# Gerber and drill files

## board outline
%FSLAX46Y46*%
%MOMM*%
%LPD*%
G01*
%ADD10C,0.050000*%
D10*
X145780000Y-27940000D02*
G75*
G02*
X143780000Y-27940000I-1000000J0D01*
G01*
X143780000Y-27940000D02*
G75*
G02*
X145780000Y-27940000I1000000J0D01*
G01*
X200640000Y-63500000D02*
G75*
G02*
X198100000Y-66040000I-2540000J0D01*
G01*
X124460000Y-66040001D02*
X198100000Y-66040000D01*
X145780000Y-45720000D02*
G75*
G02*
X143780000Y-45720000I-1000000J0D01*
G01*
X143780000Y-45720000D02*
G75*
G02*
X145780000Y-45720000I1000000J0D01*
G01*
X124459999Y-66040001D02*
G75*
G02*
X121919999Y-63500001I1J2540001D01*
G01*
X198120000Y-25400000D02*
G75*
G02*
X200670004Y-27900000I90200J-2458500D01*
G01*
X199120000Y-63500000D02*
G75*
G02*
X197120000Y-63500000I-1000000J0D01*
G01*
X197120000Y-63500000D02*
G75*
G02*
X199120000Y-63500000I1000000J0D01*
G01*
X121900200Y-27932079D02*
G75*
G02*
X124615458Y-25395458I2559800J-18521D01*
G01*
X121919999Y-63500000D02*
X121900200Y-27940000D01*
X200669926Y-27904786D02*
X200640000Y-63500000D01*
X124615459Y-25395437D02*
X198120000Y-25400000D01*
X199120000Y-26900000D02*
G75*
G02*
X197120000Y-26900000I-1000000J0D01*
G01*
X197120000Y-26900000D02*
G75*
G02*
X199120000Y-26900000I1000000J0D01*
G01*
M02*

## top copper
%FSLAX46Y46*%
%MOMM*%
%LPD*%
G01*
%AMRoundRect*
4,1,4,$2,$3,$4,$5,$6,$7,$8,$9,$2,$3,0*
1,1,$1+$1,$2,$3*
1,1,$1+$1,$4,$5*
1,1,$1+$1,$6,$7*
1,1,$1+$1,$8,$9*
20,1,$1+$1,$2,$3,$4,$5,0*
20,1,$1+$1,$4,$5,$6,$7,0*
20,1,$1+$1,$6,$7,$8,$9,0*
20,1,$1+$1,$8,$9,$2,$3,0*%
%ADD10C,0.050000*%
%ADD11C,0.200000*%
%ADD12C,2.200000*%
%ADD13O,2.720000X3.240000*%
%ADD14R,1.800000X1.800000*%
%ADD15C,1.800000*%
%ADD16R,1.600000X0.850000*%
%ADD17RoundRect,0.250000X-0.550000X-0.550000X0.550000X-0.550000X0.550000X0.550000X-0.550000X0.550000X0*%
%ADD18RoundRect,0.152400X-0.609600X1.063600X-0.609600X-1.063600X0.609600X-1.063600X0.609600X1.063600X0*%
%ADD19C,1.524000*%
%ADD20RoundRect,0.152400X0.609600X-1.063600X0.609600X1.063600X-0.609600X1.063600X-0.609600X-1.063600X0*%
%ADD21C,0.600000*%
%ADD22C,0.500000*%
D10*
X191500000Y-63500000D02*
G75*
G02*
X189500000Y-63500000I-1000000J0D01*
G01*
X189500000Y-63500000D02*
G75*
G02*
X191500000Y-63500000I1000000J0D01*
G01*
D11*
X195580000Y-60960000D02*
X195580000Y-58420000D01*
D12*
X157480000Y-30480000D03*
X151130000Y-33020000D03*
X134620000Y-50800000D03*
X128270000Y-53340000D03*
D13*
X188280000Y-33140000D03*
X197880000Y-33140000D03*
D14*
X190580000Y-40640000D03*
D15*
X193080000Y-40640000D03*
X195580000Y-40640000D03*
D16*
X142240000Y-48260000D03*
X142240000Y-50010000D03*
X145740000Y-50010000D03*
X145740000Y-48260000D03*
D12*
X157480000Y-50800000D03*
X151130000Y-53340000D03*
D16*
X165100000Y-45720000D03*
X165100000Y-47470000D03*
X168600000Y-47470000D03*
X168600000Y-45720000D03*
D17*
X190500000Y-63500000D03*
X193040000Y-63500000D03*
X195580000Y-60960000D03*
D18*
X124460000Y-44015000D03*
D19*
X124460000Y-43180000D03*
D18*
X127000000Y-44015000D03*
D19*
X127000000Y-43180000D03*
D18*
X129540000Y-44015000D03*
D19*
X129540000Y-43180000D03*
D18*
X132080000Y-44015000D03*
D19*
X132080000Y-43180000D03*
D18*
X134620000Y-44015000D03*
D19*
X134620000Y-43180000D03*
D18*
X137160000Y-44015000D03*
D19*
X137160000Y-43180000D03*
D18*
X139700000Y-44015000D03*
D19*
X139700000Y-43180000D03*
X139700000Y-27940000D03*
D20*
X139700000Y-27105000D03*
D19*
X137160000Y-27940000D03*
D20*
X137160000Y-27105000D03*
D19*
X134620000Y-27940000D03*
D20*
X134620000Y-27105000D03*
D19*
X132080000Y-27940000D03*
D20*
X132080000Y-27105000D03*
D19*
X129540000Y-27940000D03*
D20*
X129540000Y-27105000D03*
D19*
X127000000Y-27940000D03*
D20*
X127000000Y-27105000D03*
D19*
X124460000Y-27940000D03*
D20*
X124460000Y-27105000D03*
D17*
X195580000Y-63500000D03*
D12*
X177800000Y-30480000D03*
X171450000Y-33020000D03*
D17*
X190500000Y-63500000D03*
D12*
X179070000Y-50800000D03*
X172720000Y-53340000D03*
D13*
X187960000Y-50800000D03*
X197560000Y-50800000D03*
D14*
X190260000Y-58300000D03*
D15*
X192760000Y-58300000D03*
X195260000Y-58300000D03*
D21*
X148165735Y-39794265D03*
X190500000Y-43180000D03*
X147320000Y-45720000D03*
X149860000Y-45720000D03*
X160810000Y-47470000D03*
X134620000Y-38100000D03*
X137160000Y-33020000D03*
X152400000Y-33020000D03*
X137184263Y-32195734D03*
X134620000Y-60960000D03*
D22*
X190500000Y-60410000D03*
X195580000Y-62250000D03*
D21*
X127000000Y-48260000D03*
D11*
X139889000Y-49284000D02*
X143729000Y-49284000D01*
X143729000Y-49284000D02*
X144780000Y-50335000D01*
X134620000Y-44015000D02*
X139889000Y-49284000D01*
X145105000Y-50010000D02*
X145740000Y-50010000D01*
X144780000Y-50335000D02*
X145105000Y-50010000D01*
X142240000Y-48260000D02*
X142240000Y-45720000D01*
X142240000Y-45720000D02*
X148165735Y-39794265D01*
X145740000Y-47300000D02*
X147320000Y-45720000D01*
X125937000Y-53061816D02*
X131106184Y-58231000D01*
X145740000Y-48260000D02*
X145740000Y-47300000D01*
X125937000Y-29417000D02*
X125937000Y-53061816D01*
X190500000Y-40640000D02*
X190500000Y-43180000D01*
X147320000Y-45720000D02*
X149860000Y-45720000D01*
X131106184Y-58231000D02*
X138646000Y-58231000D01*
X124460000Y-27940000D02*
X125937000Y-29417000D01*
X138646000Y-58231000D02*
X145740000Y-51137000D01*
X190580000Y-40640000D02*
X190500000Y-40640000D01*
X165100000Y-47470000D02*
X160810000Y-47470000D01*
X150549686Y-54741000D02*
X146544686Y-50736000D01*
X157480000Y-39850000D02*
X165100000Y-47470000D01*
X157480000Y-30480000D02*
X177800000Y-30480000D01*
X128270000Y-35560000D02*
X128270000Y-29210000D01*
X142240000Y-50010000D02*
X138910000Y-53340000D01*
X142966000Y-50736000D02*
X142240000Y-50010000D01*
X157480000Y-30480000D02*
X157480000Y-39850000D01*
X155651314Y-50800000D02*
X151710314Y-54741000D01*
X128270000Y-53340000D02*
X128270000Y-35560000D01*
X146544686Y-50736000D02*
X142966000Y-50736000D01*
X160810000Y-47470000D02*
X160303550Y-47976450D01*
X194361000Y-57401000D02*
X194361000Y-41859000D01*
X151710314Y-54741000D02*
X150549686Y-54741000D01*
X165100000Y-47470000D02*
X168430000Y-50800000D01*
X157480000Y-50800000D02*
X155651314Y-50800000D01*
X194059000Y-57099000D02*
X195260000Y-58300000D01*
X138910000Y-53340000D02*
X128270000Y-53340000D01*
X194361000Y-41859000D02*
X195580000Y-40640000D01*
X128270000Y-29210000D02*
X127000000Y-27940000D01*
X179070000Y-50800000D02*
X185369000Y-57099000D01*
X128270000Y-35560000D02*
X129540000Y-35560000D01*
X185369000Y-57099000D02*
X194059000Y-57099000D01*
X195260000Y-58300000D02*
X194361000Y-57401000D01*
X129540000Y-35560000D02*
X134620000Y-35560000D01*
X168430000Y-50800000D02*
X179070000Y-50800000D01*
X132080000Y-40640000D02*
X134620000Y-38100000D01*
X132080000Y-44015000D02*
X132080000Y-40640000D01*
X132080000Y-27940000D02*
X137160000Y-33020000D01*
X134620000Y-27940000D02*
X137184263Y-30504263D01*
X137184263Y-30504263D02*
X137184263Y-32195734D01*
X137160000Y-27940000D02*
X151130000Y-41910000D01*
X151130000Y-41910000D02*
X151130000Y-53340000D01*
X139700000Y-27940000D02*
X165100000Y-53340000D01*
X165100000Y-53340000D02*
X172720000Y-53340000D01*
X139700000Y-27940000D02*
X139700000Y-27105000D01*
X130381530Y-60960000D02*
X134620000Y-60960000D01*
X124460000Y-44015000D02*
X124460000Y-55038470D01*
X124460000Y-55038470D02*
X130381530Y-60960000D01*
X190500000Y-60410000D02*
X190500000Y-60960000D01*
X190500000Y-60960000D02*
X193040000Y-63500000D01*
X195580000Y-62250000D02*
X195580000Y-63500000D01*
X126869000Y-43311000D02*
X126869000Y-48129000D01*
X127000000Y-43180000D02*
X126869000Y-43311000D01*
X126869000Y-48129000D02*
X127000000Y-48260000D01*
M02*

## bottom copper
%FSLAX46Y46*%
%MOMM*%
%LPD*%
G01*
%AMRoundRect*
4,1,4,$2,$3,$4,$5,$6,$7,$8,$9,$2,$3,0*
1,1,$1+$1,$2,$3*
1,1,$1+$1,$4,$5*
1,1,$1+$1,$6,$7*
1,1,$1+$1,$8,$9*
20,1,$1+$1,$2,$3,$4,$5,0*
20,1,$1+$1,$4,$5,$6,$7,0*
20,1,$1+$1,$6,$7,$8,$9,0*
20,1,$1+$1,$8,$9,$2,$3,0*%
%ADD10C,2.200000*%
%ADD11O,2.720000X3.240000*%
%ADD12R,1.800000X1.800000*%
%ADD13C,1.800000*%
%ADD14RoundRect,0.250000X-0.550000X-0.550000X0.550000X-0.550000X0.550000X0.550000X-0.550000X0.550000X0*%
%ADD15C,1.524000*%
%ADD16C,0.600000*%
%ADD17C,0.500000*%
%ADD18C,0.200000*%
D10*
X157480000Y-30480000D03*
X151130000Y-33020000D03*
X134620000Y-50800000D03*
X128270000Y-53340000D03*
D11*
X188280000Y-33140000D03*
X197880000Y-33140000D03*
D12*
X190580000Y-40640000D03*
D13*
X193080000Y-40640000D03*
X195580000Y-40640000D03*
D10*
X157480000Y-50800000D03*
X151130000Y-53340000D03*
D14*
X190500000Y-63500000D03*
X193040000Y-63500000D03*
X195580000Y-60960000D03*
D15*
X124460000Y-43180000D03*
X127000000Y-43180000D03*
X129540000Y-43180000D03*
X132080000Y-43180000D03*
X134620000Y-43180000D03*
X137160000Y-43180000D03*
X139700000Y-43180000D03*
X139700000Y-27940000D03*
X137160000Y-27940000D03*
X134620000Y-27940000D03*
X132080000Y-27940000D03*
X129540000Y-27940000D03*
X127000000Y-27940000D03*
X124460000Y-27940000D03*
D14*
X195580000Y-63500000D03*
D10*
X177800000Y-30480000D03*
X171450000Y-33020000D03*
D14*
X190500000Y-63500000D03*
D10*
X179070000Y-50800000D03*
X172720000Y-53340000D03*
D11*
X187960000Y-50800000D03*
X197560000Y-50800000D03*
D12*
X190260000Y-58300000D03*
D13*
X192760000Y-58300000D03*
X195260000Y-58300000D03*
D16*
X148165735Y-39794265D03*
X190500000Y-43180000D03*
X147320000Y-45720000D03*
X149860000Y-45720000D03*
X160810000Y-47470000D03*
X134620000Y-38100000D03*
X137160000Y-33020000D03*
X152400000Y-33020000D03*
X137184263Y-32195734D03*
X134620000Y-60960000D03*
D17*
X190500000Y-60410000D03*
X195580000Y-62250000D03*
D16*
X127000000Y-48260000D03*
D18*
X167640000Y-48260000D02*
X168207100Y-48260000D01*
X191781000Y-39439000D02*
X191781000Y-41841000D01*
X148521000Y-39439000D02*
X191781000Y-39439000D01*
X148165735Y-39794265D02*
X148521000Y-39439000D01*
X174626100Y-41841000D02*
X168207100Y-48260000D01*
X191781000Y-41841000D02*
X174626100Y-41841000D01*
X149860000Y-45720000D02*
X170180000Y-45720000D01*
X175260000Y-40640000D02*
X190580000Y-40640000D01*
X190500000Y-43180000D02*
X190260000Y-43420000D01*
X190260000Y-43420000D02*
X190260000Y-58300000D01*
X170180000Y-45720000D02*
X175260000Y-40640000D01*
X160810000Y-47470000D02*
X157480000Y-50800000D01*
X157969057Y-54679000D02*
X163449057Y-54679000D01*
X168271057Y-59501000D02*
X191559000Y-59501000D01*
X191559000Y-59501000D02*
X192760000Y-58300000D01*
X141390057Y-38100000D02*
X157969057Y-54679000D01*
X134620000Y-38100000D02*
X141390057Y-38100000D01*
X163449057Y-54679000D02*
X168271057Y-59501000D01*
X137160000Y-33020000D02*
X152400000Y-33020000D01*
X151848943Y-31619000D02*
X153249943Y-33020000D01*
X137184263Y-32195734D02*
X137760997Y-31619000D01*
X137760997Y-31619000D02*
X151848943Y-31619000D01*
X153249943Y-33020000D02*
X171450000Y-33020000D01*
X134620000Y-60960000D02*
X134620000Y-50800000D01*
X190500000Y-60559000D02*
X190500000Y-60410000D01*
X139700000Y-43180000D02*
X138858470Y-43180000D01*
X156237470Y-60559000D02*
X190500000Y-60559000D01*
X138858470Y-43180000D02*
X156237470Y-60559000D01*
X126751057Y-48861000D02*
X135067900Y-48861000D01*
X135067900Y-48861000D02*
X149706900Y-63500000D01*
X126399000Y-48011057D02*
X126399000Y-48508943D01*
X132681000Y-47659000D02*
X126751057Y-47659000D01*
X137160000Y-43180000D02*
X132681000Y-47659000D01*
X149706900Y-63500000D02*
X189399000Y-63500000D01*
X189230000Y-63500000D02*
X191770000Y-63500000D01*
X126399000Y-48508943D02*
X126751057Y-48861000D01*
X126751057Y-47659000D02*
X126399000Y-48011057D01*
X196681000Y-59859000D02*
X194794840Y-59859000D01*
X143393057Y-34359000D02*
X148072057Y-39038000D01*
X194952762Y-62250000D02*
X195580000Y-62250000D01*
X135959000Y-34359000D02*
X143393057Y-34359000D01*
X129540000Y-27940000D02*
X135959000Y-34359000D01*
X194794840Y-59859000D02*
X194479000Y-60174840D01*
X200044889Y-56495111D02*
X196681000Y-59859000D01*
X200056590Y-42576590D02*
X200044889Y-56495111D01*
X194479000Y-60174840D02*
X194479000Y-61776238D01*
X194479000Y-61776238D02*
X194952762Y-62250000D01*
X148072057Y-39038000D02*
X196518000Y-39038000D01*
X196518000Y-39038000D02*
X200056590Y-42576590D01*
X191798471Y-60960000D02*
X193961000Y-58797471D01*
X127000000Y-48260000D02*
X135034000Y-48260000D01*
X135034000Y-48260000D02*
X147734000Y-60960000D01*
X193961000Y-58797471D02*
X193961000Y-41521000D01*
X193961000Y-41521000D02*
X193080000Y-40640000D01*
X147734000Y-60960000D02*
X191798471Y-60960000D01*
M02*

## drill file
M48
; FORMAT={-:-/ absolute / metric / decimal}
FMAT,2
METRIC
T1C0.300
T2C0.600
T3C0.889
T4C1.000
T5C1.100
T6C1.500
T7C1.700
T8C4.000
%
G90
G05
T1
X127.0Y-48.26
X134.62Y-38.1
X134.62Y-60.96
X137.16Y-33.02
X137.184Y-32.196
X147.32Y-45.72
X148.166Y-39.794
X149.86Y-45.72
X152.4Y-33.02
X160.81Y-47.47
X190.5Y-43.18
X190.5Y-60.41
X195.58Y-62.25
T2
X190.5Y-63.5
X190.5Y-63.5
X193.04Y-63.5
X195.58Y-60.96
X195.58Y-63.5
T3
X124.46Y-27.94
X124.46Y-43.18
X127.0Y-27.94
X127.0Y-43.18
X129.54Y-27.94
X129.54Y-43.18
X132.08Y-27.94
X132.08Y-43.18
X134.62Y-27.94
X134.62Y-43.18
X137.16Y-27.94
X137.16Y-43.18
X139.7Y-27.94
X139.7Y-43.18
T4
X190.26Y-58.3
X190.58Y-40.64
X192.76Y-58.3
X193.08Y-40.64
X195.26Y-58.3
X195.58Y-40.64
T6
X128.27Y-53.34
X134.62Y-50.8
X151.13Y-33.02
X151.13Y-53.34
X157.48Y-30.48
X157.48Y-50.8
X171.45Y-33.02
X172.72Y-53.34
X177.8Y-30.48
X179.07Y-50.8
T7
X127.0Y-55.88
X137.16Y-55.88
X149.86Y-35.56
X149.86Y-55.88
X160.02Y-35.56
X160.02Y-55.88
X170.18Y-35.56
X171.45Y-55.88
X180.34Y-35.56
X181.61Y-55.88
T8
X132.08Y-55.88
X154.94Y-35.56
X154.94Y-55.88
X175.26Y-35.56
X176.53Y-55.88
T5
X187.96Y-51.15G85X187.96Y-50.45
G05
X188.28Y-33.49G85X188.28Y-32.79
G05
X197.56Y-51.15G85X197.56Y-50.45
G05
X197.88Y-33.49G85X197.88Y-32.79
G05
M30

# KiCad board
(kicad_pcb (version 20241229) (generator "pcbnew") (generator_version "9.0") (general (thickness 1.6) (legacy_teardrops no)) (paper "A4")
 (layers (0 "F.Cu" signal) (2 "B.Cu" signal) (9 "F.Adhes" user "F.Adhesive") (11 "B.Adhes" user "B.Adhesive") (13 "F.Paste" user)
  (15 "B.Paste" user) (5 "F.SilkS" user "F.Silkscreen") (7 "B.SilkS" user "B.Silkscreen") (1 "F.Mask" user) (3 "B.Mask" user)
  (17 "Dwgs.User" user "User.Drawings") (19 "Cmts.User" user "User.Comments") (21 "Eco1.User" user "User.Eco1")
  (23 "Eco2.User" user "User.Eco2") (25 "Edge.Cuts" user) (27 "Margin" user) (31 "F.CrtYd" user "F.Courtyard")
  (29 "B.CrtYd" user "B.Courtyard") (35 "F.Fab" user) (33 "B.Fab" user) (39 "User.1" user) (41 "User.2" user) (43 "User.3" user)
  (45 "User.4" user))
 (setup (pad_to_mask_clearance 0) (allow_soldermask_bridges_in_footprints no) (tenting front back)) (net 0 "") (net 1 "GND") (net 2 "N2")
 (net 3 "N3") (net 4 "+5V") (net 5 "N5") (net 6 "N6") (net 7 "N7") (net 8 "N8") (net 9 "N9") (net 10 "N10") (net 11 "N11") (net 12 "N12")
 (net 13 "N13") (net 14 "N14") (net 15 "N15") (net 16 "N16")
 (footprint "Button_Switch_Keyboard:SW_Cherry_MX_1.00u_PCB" (layer "F.Cu") (at 157.48 30.48)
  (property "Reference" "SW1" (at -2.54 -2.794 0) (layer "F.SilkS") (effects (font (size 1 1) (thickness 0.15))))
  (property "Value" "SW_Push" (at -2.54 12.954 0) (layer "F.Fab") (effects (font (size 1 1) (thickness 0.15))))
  (pad "" np_thru_hole circle (at -7.62 5.08) (size 1.7 1.7) (drill 1.7) (layers "*.Cu" "*.Mask"))
  (pad "" np_thru_hole circle (at -2.54 5.08) (size 4 4) (drill 4) (layers "*.Cu" "*.Mask"))
  (pad "" np_thru_hole circle (at 2.54 5.08) (size 1.7 1.7) (drill 1.7) (layers "*.Cu" "*.Mask"))
  (pad "1" thru_hole circle (at 0 0) (size 2.2 2.2) (drill 1.5) (layers "*.Cu" "*.Mask") (remove_unused_layers no) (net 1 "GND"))
  (pad "2" thru_hole circle (at -6.35 2.54) (size 2.2 2.2) (drill 1.5) (layers "*.Cu" "*.Mask") (remove_unused_layers no) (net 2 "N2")))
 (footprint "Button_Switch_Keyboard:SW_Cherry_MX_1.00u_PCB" (layer "F.Cu") (at 134.62 50.8)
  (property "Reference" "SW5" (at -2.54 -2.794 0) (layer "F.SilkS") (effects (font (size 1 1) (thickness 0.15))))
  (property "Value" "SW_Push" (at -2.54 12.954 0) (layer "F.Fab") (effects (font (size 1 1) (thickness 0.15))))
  (pad "" np_thru_hole circle (at -7.62 5.08) (size 1.7 1.7) (drill 1.7) (layers "*.Cu" "*.Mask"))
  (pad "" np_thru_hole circle (at -2.54 5.08) (size 4 4) (drill 4) (layers "*.Cu" "*.Mask"))
  (pad "" np_thru_hole circle (at 2.54 5.08) (size 1.7 1.7) (drill 1.7) (layers "*.Cu" "*.Mask"))
  (pad "1" thru_hole circle (at 0 0) (size 2.2 2.2) (drill 1.5) (layers "*.Cu" "*.Mask") (remove_unused_layers no) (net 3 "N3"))
  (pad "2" thru_hole circle (at -6.35 2.54) (size 2.2 2.2) (drill 1.5) (layers "*.Cu" "*.Mask") (remove_unused_layers no) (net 1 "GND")))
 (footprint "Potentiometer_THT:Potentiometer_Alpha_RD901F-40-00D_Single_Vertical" (layer "F.Cu") (at 190.58 40.64 90)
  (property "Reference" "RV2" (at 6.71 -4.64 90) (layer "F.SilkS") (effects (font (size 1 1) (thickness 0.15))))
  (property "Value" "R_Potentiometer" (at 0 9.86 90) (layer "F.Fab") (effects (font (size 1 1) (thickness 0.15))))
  (pad "" thru_hole oval (at 7.5 -2.3 180) (size 2.72 3.24) (drill oval 1.1 1.8) (layers "*.Cu" "*.Mask") (remove_unused_layers no))
  (pad "" thru_hole oval (at 7.5 7.3 180) (size 2.72 3.24) (drill oval 1.1 1.8) (layers "*.Cu" "*.Mask") (remove_unused_layers no))
  (pad "1" thru_hole rect (at 0 0 180) (size 1.8 1.8) (drill 1) (layers "*.Cu" "*.Mask") (remove_unused_layers no) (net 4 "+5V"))
  (pad "2" thru_hole circle (at 0 2.5 180) (size 1.8 1.8) (drill 1) (layers "*.Cu" "*.Mask") (remove_unused_layers no) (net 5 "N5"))
  (pad "3" thru_hole circle (at 0 5 180) (size 1.8 1.8) (drill 1) (layers "*.Cu" "*.Mask") (remove_unused_layers no) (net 1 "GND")))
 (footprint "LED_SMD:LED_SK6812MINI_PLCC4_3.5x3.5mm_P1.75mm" (layer "F.Cu") (at 143.99 49.135)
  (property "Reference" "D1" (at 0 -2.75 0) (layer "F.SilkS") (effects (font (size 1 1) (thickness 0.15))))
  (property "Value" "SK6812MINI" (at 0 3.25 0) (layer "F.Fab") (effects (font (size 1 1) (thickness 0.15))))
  (pad "1" smd rect (at -1.75 -0.875) (size 1.6 0.85) (layers "F.Cu" "F.Mask" "F.Paste") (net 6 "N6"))
  (pad "2" smd rect (at -1.75 0.875) (size 1.6 0.85) (layers "F.Cu" "F.Mask" "F.Paste") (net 1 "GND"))
  (pad "3" smd rect (at 1.75 0.875) (size 1.6 0.85) (layers "F.Cu" "F.Mask" "F.Paste") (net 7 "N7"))
  (pad "4" smd rect (at 1.75 -0.875) (size 1.6 0.85) (layers "F.Cu" "F.Mask" "F.Paste") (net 4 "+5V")))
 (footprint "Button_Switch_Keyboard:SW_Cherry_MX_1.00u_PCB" (layer "F.Cu") (at 157.48 50.8)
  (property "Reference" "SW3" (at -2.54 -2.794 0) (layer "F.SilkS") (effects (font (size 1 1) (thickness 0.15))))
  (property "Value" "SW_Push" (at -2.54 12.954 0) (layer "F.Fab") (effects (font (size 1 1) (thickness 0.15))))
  (pad "" np_thru_hole circle (at -7.62 5.08) (size 1.7 1.7) (drill 1.7) (layers "*.Cu" "*.Mask"))
  (pad "" np_thru_hole circle (at -2.54 5.08) (size 4 4) (drill 4) (layers "*.Cu" "*.Mask"))
  (pad "" np_thru_hole circle (at 2.54 5.08) (size 1.7 1.7) (drill 1.7) (layers "*.Cu" "*.Mask"))
  (pad "1" thru_hole circle (at 0 0) (size 2.2 2.2) (drill 1.5) (layers "*.Cu" "*.Mask") (remove_unused_layers no) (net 1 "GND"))
  (pad "2" thru_hole circle (at -6.35 2.54) (size 2.2 2.2) (drill 1.5) (layers "*.Cu" "*.Mask") (remove_unused_layers no) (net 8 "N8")))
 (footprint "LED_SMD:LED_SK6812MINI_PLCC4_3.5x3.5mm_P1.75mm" (layer "F.Cu") (at 166.85 46.595)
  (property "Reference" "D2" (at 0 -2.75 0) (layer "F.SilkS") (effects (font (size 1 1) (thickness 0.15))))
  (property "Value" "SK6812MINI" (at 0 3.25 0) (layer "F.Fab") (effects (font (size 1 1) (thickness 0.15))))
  (pad "1" smd rect (at -1.75 -0.875) (size 1.6 0.85) (layers "F.Cu" "F.Mask" "F.Paste") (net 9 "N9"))
  (pad "2" smd rect (at -1.75 0.875) (size 1.6 0.85) (layers "F.Cu" "F.Mask" "F.Paste") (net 1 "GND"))
  (pad "3" smd rect (at 1.75 0.875) (size 1.6 0.85) (layers "F.Cu" "F.Mask" "F.Paste") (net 6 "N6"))
  (pad "4" smd rect (at 1.75 -0.875) (size 1.6 0.85) (layers "F.Cu" "F.Mask" "F.Paste") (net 4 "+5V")))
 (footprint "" (layer "F.Cu") (at 190.5 63.5)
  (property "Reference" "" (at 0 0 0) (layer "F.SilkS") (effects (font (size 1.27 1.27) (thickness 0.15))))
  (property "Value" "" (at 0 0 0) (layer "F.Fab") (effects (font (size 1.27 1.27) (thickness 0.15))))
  (pad "1" thru_hole roundrect (at 0 0) (size 1.6 1.6) (drill 0.6) (layers "*.Cu" "*.Mask") (remove_unused_layers no)
   (roundrect_rratio 0.15625)))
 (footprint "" (layer "F.Cu") (at 193.04 63.5)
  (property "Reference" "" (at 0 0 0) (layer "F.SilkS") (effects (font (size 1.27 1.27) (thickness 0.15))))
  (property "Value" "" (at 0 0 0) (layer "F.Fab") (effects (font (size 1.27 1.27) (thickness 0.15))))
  (pad "1" thru_hole roundrect (at 0 0) (size 1.6 1.6) (drill 0.6) (layers "*.Cu" "*.Mask") (remove_unused_layers no)
   (roundrect_rratio 0.15625)))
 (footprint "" (layer "F.Cu") (at 195.58 60.96)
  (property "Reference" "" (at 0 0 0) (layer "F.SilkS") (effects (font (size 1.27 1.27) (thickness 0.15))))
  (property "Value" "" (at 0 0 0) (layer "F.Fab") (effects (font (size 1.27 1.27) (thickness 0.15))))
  (pad "1" thru_hole roundrect (at 0 0) (size 1.6 1.6) (drill 0.6) (layers "*.Cu" "*.Mask") (remove_unused_layers no)
   (roundrect_rratio 0.15625)))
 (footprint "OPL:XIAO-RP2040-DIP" (layer "F.Cu") (at 132.08 35.56 90)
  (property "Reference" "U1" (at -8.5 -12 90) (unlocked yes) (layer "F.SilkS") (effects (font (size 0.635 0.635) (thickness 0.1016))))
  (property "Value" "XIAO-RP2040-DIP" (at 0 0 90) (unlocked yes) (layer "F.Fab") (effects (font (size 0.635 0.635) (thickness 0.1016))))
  (pad "1" smd roundrect (at -8.455 -7.62 270) (size 2.432 1.524) (layers "F.Cu" "F.Mask") (roundrect_rratio 0.1) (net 3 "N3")
   (thermal_bridge_angle 45))
  (pad "1" thru_hole circle (at -7.62 -7.62 270) (size 1.524 1.524) (drill 0.889) (layers "*.Cu" "*.Mask") (remove_unused_layers no)
   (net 3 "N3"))
  (pad "2" smd roundrect (at -8.455 -5.08 270) (size 2.432 1.524) (layers "F.Cu" "F.Mask") (roundrect_rratio 0.1) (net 5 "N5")
   (thermal_bridge_angle 45))
  (pad "2" thru_hole circle (at -7.62 -5.08 270) (size 1.524 1.524) (drill 0.889) (layers "*.Cu" "*.Mask") (remove_unused_layers no)
   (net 5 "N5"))
  (pad "3" smd roundrect (at -8.455 -2.54 270) (size 2.432 1.524) (layers "F.Cu" "F.Mask") (roundrect_rratio 0.1) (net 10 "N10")
   (thermal_bridge_angle 45))
  (pad "3" thru_hole circle (at -7.62 -2.54 270) (size 1.524 1.524) (drill 0.889) (layers "*.Cu" "*.Mask") (remove_unused_layers no)
   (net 10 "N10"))
  (pad "4" smd roundrect (at -8.455 0 270) (size 2.432 1.524) (layers "F.Cu" "F.Mask") (roundrect_rratio 0.1) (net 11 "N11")
   (thermal_bridge_angle 45))
  (pad "4" thru_hole circle (at -7.62 0 270) (size 1.524 1.524) (drill 0.889) (layers "*.Cu" "*.Mask") (remove_unused_layers no)
   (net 11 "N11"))
  (pad "5" smd roundrect (at -8.455 2.54 270) (size 2.432 1.524) (layers "F.Cu" "F.Mask") (roundrect_rratio 0.1) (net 7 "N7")
   (thermal_bridge_angle 45))
  (pad "5" thru_hole circle (at -7.62 2.54 270) (size 1.524 1.524) (drill 0.889) (layers "*.Cu" "*.Mask") (remove_unused_layers no)
   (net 7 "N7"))
  (pad "6" smd roundrect (at -8.455 5.08 270) (size 2.432 1.524) (layers "F.Cu" "F.Mask") (roundrect_rratio 0.1) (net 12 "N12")
   (thermal_bridge_angle 45))
  (pad "6" thru_hole circle (at -7.62 5.08 270) (size 1.524 1.524) (drill 0.889) (layers "*.Cu" "*.Mask") (remove_unused_layers no)
   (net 12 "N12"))
  (pad "7" smd roundrect (at -8.455 7.62 270) (size 2.432 1.524) (layers "F.Cu" "F.Mask") (roundrect_rratio 0.1) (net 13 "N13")
   (thermal_bridge_angle 45))
  (pad "7" thru_hole circle (at -7.62 7.62 270) (size 1.524 1.524) (drill 0.889) (layers "*.Cu" "*.Mask") (remove_unused_layers no)
   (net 13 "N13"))
  (pad "8" thru_hole circle (at 7.62 7.62 90) (size 1.524 1.524) (drill 0.889) (layers "*.Cu" "*.Mask") (remove_unused_layers no)
   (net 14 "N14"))
  (pad "8" smd roundrect (at 8.455 7.62 90) (size 2.432 1.524) (layers "F.Cu" "F.Mask") (roundrect_rratio 0.1) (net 14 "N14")
   (thermal_bridge_angle 45))
  (pad "9" thru_hole circle (at 7.62 5.08 90) (size 1.524 1.524) (drill 0.889) (layers "*.Cu" "*.Mask") (remove_unused_layers no)
   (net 8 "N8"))
  (pad "9" smd roundrect (at 8.455 5.08 90) (size 2.432 1.524) (layers "F.Cu" "F.Mask") (roundrect_rratio 0.1) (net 8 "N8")
   (thermal_bridge_angle 45))
  (pad "10" thru_hole circle (at 7.62 2.54 90) (size 1.524 1.524) (drill 0.889) (layers "*.Cu" "*.Mask") (remove_unused_layers no)
   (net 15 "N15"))
  (pad "10" smd roundrect (at 8.455 2.54 90) (size 2.432 1.524) (layers "F.Cu" "F.Mask") (roundrect_rratio 0.1) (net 15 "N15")
   (thermal_bridge_angle 45))
  (pad "11" thru_hole circle (at 7.62 0 90) (size 1.524 1.524) (drill 0.889) (layers "*.Cu" "*.Mask") (remove_unused_layers no) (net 2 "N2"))
  (pad "11" smd roundrect (at 8.455 0 90) (size 2.432 1.524) (layers "F.Cu" "F.Mask") (roundrect_rratio 0.1) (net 2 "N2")
   (thermal_bridge_angle 45))
  (pad "12" thru_hole circle (at 7.62 -2.54 90) (size 1.524 1.524) (drill 0.889) (layers "*.Cu" "*.Mask") (remove_unused_layers no)
   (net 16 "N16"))
  (pad "12" smd roundrect (at 8.455 -2.54 90) (size 2.432 1.524) (layers "F.Cu" "F.Mask") (roundrect_rratio 0.1) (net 16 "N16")
   (thermal_bridge_angle 45))
  (pad "13" thru_hole circle (at 7.62 -5.08 90) (size 1.524 1.524) (drill 0.889) (layers "*.Cu" "*.Mask") (remove_unused_layers no)
   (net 1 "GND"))
  (pad "13" smd roundrect (at 8.455 -5.08 90) (size 2.432 1.524) (layers "F.Cu" "F.Mask") (roundrect_rratio 0.1) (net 1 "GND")
   (thermal_bridge_angle 45))
  (pad "14" thru_hole circle (at 7.62 -7.62 90) (size 1.524 1.524) (drill 0.889) (layers "*.Cu" "*.Mask") (remove_unused_layers no)
   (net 4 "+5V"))
  (pad "14" smd roundrect (at 8.455 -7.62 90) (size 2.432 1.524) (layers "F.Cu" "F.Mask") (roundrect_rratio 0.1) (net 4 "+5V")
   (thermal_bridge_angle 45)))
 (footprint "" (layer "F.Cu") (at 195.58 63.5)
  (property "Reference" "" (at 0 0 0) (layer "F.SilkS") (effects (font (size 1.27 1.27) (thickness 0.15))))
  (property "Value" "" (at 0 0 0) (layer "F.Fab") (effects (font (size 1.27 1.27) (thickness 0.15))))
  (pad "1" thru_hole roundrect (at 0 0) (size 1.6 1.6) (drill 0.6) (layers "*.Cu" "*.Mask") (remove_unused_layers no)
   (roundrect_rratio 0.15625)))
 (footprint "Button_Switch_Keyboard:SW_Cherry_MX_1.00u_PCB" (layer "F.Cu") (at 177.8 30.48)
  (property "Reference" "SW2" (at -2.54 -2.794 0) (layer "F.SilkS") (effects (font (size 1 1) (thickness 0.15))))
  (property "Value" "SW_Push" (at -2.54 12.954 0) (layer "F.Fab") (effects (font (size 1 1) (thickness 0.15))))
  (pad "" np_thru_hole circle (at -7.62 5.08) (size 1.7 1.7) (drill 1.7) (layers "*.Cu" "*.Mask"))
  (pad "" np_thru_hole circle (at -2.54 5.08) (size 4 4) (drill 4) (layers "*.Cu" "*.Mask"))
  (pad "" np_thru_hole circle (at 2.54 5.08) (size 1.7 1.7) (drill 1.7) (layers "*.Cu" "*.Mask"))
  (pad "1" thru_hole circle (at 0 0) (size 2.2 2.2) (drill 1.5) (layers "*.Cu" "*.Mask") (remove_unused_layers no) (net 1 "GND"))
  (pad "2" thru_hole circle (at -6.35 2.54) (size 2.2 2.2) (drill 1.5) (layers "*.Cu" "*.Mask") (remove_unused_layers no) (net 15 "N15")))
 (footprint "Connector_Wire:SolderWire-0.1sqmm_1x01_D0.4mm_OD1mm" (layer "F.Cu") (at 190.5 63.5)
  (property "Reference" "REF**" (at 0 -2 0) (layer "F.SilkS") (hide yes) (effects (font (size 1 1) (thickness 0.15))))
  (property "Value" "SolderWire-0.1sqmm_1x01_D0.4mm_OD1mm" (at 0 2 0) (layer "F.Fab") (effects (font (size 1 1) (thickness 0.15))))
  (pad "1" thru_hole roundrect (at 0 0) (size 1.6 1.6) (drill 0.6) (layers "*.Cu" "*.Mask") (remove_unused_layers no)
   (roundrect_rratio 0.15625)))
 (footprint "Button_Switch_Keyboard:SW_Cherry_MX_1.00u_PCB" (layer "F.Cu") (at 179.07 50.8)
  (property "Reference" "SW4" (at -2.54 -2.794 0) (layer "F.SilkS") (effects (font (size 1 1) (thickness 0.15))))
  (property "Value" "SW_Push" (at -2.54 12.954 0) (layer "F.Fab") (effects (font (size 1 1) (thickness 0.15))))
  (pad "" np_thru_hole circle (at -7.62 5.08) (size 1.7 1.7) (drill 1.7) (layers "*.Cu" "*.Mask"))
  (pad "" np_thru_hole circle (at -2.54 5.08) (size 4 4) (drill 4) (layers "*.Cu" "*.Mask"))
  (pad "" np_thru_hole circle (at 2.54 5.08) (size 1.7 1.7) (drill 1.7) (layers "*.Cu" "*.Mask"))
  (pad "1" thru_hole circle (at 0 0) (size 2.2 2.2) (drill 1.5) (layers "*.Cu" "*.Mask") (remove_unused_layers no) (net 1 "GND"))
  (pad "2" thru_hole circle (at -6.35 2.54) (size 2.2 2.2) (drill 1.5) (layers "*.Cu" "*.Mask") (remove_unused_layers no) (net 14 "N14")))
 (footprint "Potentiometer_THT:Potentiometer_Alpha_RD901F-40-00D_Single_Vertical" (layer "F.Cu") (at 190.26 58.3 90)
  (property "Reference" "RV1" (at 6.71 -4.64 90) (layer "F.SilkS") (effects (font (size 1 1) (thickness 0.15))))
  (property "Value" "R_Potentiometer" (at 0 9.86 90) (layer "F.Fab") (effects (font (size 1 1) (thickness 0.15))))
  (pad "" thru_hole oval (at 7.5 -2.3 180) (size 2.72 3.24) (drill oval 1.1 1.8) (layers "*.Cu" "*.Mask") (remove_unused_layers no))
  (pad "" thru_hole oval (at 7.5 7.3 180) (size 2.72 3.24) (drill oval 1.1 1.8) (layers "*.Cu" "*.Mask") (remove_unused_layers no))
  (pad "1" thru_hole rect (at 0 0 180) (size 1.8 1.8) (drill 1) (layers "*.Cu" "*.Mask") (remove_unused_layers no) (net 4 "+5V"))
  (pad "2" thru_hole circle (at 0 2.5 180) (size 1.8 1.8) (drill 1) (layers "*.Cu" "*.Mask") (remove_unused_layers no) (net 11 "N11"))
  (pad "3" thru_hole circle (at 0 5 180) (size 1.8 1.8) (drill 1) (layers "*.Cu" "*.Mask") (remove_unused_layers no) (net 1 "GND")))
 (gr_circle (center 190.5 63.5) (end 191.5 63.5) (stroke (width 0.05) (type solid)) (fill no) (layer "F.Cu") (net 12))
 (gr_line (start 195.58 60.96) (end 195.58 58.42) (stroke (width 0.2) (type default)) (layer "F.Cu") (net 1))
 (gr_circle (center 144.78 27.94) (end 145.78 27.94) (stroke (width 0.05) (type solid)) (fill no) (layer "Edge.Cuts"))
 (gr_arc (start 200.64 63.5) (mid 199.896051 65.296051) (end 198.1 66.04) (stroke (width 0.05) (type solid)) (layer "Edge.Cuts"))
 (gr_line (start 124.46 66.040001) (end 198.1 66.04) (stroke (width 0.05) (type default)) (layer "Edge.Cuts"))
 (gr_circle (center 144.78 45.72) (end 145.78 45.72) (stroke (width 0.05) (type solid)) (fill no) (layer "Edge.Cuts"))
 (gr_arc (start 124.459999 66.040001) (mid 122.663948 65.296052) (end 121.919999 63.500001) (stroke (width 0.05) (type solid))
  (layer "Edge.Cuts"))
 (gr_arc (start 198.12 25.4) (mid 199.920193 26.089807) (end 200.67 27.9) (stroke (width 0.05) (type solid)) (layer "Edge.Cuts"))
 (gr_circle (center 198.12 63.5) (end 199.12 63.5) (stroke (width 0.05) (type solid)) (fill no) (layer "Edge.Cuts"))
 (gr_arc (start 121.9002 27.932079) (mid 122.712473 26.08) (end 124.615459 25.395437) (stroke (width 0.05) (type solid)) (layer "Edge.Cuts"))
 (gr_line (start 121.919999 63.5) (end 121.9002 27.94) (stroke (width 0.05) (type default)) (layer "Edge.Cuts"))
 (gr_line (start 200.669926 27.904786) (end 200.64 63.5) (stroke (width 0.05) (type default)) (layer "Edge.Cuts"))
 (gr_line (start 124.615459 25.395437) (end 198.12 25.4) (stroke (width 0.05) (type default)) (layer "Edge.Cuts"))
 (gr_circle (center 198.12 26.9) (end 199.12 26.9) (stroke (width 0.05) (type solid)) (fill no) (layer "Edge.Cuts"))
 (segment (start 139.889 49.284) (end 143.729 49.284) (width 0.2) (layer "F.Cu") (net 7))
 (segment (start 143.729 49.284) (end 144.78 50.335) (width 0.2) (layer "F.Cu") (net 7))
 (segment (start 134.62 44.015) (end 139.889 49.284) (width 0.2) (layer "F.Cu") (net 7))
 (segment (start 145.105 50.01) (end 145.74 50.01) (width 0.2) (layer "F.Cu") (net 7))
 (segment (start 144.78 50.335) (end 145.105 50.01) (width 0.2) (layer "F.Cu") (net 7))
 (segment (start 142.24 48.26) (end 142.24 45.72) (width 0.2) (layer "F.Cu") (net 6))
 (segment (start 142.24 45.72) (end 148.165735 39.794265) (width 0.2) (layer "F.Cu") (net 6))
 (via (at 148.165735 39.794265) (size 0.6) (drill 0.3) (layers "F.Cu" "B.Cu") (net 6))
 (segment (start 167.64 48.26) (end 168.2071 48.26) (width 0.2) (layer "B.Cu") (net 6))
 (segment (start 191.781 39.439) (end 191.781 41.841) (width 0.2) (layer "B.Cu") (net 6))
 (segment (start 148.521 39.439) (end 191.781 39.439) (width 0.2) (layer "B.Cu") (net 6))
 (segment (start 148.165735 39.794265) (end 148.521 39.439) (width 0.2) (layer "B.Cu") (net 6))
 (segment (start 174.6261 41.841) (end 168.2071 48.26) (width 0.2) (layer "B.Cu") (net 6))
 (segment (start 191.781 41.841) (end 174.6261 41.841) (width 0.2) (layer "B.Cu") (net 6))
 (segment (start 145.74 47.3) (end 147.32 45.72) (width 0.2) (layer "F.Cu") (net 4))
 (segment (start 125.937 53.061816) (end 131.106184 58.231) (width 0.2) (layer "F.Cu") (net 4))
 (segment (start 145.74 48.26) (end 145.74 47.3) (width 0.2) (layer "F.Cu") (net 4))
 (segment (start 125.937 29.417) (end 125.937 53.061816) (width 0.2) (layer "F.Cu") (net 4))
 (segment (start 190.5 40.64) (end 190.5 43.18) (width 0.2) (layer "F.Cu") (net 4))
 (segment (start 147.32 45.72) (end 149.86 45.72) (width 0.2) (layer "F.Cu") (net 4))
 (segment (start 131.106184 58.231) (end 138.646 58.231) (width 0.2) (layer "F.Cu") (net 4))
 (segment (start 124.46 27.94) (end 125.937 29.417) (width 0.2) (layer "F.Cu") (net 4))
 (segment (start 138.646 58.231) (end 145.74 51.137) (width 0.2) (layer "F.Cu") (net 4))
 (segment (start 190.58 40.64) (end 190.5 40.64) (width 0.2) (layer "F.Cu") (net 4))
 (via (at 190.5 43.18) (size 0.6) (drill 0.3) (layers "F.Cu" "B.Cu") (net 4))
 (via (at 147.32 45.72) (size 0.6) (drill 0.3) (layers "F.Cu" "B.Cu") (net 4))
 (via (at 149.86 45.72) (size 0.6) (drill 0.3) (layers "F.Cu" "B.Cu") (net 4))
 (segment (start 149.86 45.72) (end 170.18 45.72) (width 0.2) (layer "B.Cu") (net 4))
 (segment (start 175.26 40.64) (end 190.58 40.64) (width 0.2) (layer "B.Cu") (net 4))
 (segment (start 190.5 43.18) (end 190.26 43.42) (width 0.2) (layer "B.Cu") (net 4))
 (segment (start 190.26 43.42) (end 190.26 58.3) (width 0.2) (layer "B.Cu") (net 4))
 (segment (start 170.18 45.72) (end 175.26 40.64) (width 0.2) (layer "B.Cu") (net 4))
 (segment (start 165.1 47.47) (end 160.81 47.47) (width 0.2) (layer "F.Cu") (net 1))
 (segment (start 150.549686 54.741) (end 146.544686 50.736) (width 0.2) (layer "F.Cu") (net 1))
 (segment (start 157.48 39.85) (end 165.1 47.47) (width 0.2) (layer "F.Cu") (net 1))
 (segment (start 157.48 30.48) (end 177.8 30.48) (width 0.2) (layer "F.Cu") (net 1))
 (segment (start 128.27 35.56) (end 128.27 29.21) (width 0.2) (layer "F.Cu") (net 1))
 (segment (start 142.24 50.01) (end 138.91 53.34) (width 0.2) (layer "F.Cu") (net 1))
 (segment (start 142.966 50.736) (end 142.24 50.01) (width 0.2) (layer "F.Cu") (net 1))
 (segment (start 157.48 30.48) (end 157.48 39.85) (width 0.2) (layer "F.Cu") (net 1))
 (segment (start 155.651314 50.8) (end 151.710314 54.741) (width 0.2) (layer "F.Cu") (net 1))
 (segment (start 128.27 53.34) (end 128.27 35.56) (width 0.2) (layer "F.Cu") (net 1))
 (segment (start 146.544686 50.736) (end 142.966 50.736) (width 0.2) (layer "F.Cu") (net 1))
 (segment (start 160.81 47.47) (end 160.30355 47.97645) (width 0.2) (layer "F.Cu") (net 1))
 (segment (start 194.361 57.401) (end 194.361 41.859) (width 0.2) (layer "F.Cu") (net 1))
 (segment (start 151.710314 54.741) (end 150.549686 54.741) (width 0.2) (layer "F.Cu") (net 1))
 (segment (start 165.1 47.47) (end 168.43 50.8) (width 0.2) (layer "F.Cu") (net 1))
 (segment (start 157.48 50.8) (end 155.651314 50.8) (width 0.2) (layer "F.Cu") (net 1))
 (segment (start 194.059 57.099) (end 195.26 58.3) (width 0.2) (layer "F.Cu") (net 1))
 (segment (start 138.91 53.34) (end 128.27 53.34) (width 0.2) (layer "F.Cu") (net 1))
 (segment (start 194.361 41.859) (end 195.58 40.64) (width 0.2) (layer "F.Cu") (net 1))
 (segment (start 128.27 29.21) (end 127 27.94) (width 0.2) (layer "F.Cu") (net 1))
 (segment (start 179.07 50.8) (end 185.369 57.099) (width 0.2) (layer "F.Cu") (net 1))
 (segment (start 128.27 35.56) (end 129.54 35.56) (width 0.2) (layer "F.Cu") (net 1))
 (segment (start 185.369 57.099) (end 194.059 57.099) (width 0.2) (layer "F.Cu") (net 1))
 (segment (start 195.26 58.3) (end 194.361 57.401) (width 0.2) (layer "F.Cu") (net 1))
 (segment (start 129.54 35.56) (end 134.62 35.56) (width 0.2) (layer "F.Cu") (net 1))
 (segment (start 168.43 50.8) (end 179.07 50.8) (width 0.2) (layer "F.Cu") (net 1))
 (via (at 160.81 47.47) (size 0.6) (drill 0.3) (layers "F.Cu" "B.Cu") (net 1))
 (segment (start 160.81 47.47) (end 157.48 50.8) (width 0.2) (layer "B.Cu") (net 1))
 (segment (start 132.08 40.64) (end 134.62 38.1) (width 0.2) (layer "F.Cu") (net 11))
 (segment (start 132.08 44.015) (end 132.08 40.64) (width 0.2) (layer "F.Cu") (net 11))
 (via (at 134.62 38.1) (size 0.6) (drill 0.3) (layers "F.Cu" "B.Cu") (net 11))
 (segment (start 157.969057 54.679) (end 163.449057 54.679) (width 0.2) (layer "B.Cu") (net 11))
 (segment (start 168.271057 59.501) (end 191.559 59.501) (width 0.2) (layer "B.Cu") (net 11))
 (segment (start 191.559 59.501) (end 192.76 58.3) (width 0.2) (layer "B.Cu") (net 11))
 (segment (start 141.390057 38.1) (end 157.969057 54.679) (width 0.2) (layer "B.Cu") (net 11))
 (segment (start 134.62 38.1) (end 141.390057 38.1) (width 0.2) (layer "B.Cu") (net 11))
 (segment (start 163.449057 54.679) (end 168.271057 59.501) (width 0.2) (layer "B.Cu") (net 11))
 (segment (start 132.08 27.94) (end 137.16 33.02) (width 0.2) (layer "F.Cu") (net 2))
 (via (at 137.16 33.02) (size 0.6) (drill 0.3) (layers "F.Cu" "B.Cu") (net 2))
 (via (at 152.4 33.02) (size 0.6) (drill 0.3) (layers "F.Cu" "B.Cu") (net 2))
 (segment (start 137.16 33.02) (end 152.4 33.02) (width 0.2) (layer "B.Cu") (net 2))
 (segment (start 134.62 27.94) (end 137.184263 30.504263) (width 0.2) (layer "F.Cu") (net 15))
 (segment (start 137.184263 30.504263) (end 137.184263 32.195734) (width 0.2) (layer "F.Cu") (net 15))
 (via (at 137.184263 32.195734) (size 0.6) (drill 0.3) (layers "F.Cu" "B.Cu") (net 15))
 (segment (start 151.848943 31.619) (end 153.249943 33.02) (width 0.2) (layer "B.Cu") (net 15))
 (segment (start 137.184263 32.195734) (end 137.760997 31.619) (width 0.2) (layer "B.Cu") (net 15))
 (segment (start 137.760997 31.619) (end 151.848943 31.619) (width 0.2) (layer "B.Cu") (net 15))
 (segment (start 153.249943 33.02) (end 171.45 33.02) (width 0.2) (layer "B.Cu") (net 15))
 (segment (start 137.16 27.94) (end 151.13 41.91) (width 0.2) (layer "F.Cu") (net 8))
 (segment (start 151.13 41.91) (end 151.13 53.34) (width 0.2) (layer "F.Cu") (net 8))
 (segment (start 139.7 27.94) (end 165.1 53.34) (width 0.2) (layer "F.Cu") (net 14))
 (segment (start 165.1 53.34) (end 172.72 53.34) (width 0.2) (layer "F.Cu") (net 14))
 (segment (start 139.7 27.94) (end 139.7 27.105) (width 0.2) (layer "F.Cu") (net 14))
 (segment (start 130.38153 60.96) (end 134.62 60.96) (width 0.2) (layer "F.Cu") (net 3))
 (segment (start 124.46 44.015) (end 124.46 55.03847) (width 0.2) (layer "F.Cu") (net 3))
 (segment (start 124.46 55.03847) (end 130.38153 60.96) (width 0.2) (layer "F.Cu") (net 3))
 (via (at 134.62 60.96) (size 0.6) (drill 0.3) (layers "F.Cu" "B.Cu") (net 3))
 (segment (start 134.62 60.96) (end 134.62 50.8) (width 0.2) (layer "B.Cu") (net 3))
 (segment (start 190.5 60.41) (end 190.5 60.96) (width 0.2) (layer "F.Cu") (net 13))
 (segment (start 190.5 60.96) (end 193.04 63.5) (width 0.2) (layer "F.Cu") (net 13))
 (via (at 190.5 60.41) (size 0.5) (drill 0.3) (layers "F.Cu" "B.Cu") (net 13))
 (segment (start 190.5 60.559) (end 190.5 60.41) (width 0.2) (layer "B.Cu") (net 13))
 (segment (start 139.7 43.18) (end 138.85847 43.18) (width 0.2) (layer "B.Cu") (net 13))
 (segment (start 156.23747 60.559) (end 190.5 60.559) (width 0.2) (layer "B.Cu") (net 13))
 (segment (start 138.85847 43.18) (end 156.23747 60.559) (width 0.2) (layer "B.Cu") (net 13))
 (segment (start 126.751057 48.861) (end 135.0679 48.861) (width 0.2) (layer "B.Cu") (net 12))
 (segment (start 135.0679 48.861) (end 149.7069 63.5) (width 0.2) (layer "B.Cu") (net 12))
 (segment (start 126.399 48.011057) (end 126.399 48.508943) (width 0.2) (layer "B.Cu") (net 12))
 (segment (start 132.681 47.659) (end 126.751057 47.659) (width 0.2) (layer "B.Cu") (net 12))
 (segment (start 137.16 43.18) (end 132.681 47.659) (width 0.2) (layer "B.Cu") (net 12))
 (segment (start 149.7069 63.5) (end 189.399 63.5) (width 0.2) (layer "B.Cu") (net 12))
 (segment (start 189.23 63.5) (end 191.77 63.5) (width 0.2) (layer "B.Cu") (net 12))
 (segment (start 126.399 48.508943) (end 126.751057 48.861) (width 0.2) (layer "B.Cu") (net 12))
 (segment (start 126.751057 47.659) (end 126.399 48.011057) (width 0.2) (layer "B.Cu") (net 12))
 (segment (start 195.58 62.25) (end 195.58 63.5) (width 0.2) (layer "F.Cu") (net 16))
 (via (at 195.58 62.25) (size 0.5) (drill 0.3) (layers "F.Cu" "B.Cu") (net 16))
 (segment (start 196.681 59.859) (end 194.79484 59.859) (width 0.2) (layer "B.Cu") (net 16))
 (segment (start 143.393057 34.359) (end 148.072057 39.038) (width 0.2) (layer "B.Cu") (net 16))
 (segment (start 194.952762 62.25) (end 195.58 62.25) (width 0.2) (layer "B.Cu") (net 16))
 (segment (start 135.959 34.359) (end 143.393057 34.359) (width 0.2) (layer "B.Cu") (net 16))
 (segment (start 129.54 27.94) (end 135.959 34.359) (width 0.2) (layer "B.Cu") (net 16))
 (segment (start 194.79484 59.859) (end 194.479 60.17484) (width 0.2) (layer "B.Cu") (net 16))
 (segment (start 200.044889 56.495111) (end 196.681 59.859) (width 0.2) (layer "B.Cu") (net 16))
 (segment (start 200.05659 42.57659) (end 200.044889 56.495111) (width 0.2) (layer "B.Cu") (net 16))
 (segment (start 194.479 60.17484) (end 194.479 61.776238) (width 0.2) (layer "B.Cu") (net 16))
 (segment (start 194.479 61.776238) (end 194.952762 62.25) (width 0.2) (layer "B.Cu") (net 16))
 (segment (start 148.072057 39.038) (end 196.518 39.038) (width 0.2) (layer "B.Cu") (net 16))
 (segment (start 196.518 39.038) (end 200.05659 42.57659) (width 0.2) (layer "B.Cu") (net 16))
 (segment (start 126.869 43.311) (end 126.869 48.129) (width 0.2) (layer "F.Cu") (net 5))
 (segment (start 127 43.18) (end 126.869 43.311) (width 0.2) (layer "F.Cu") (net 5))
 (segment (start 126.869 48.129) (end 127 48.26) (width 0.2) (layer "F.Cu") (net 5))
 (via (at 127 48.26) (size 0.6) (drill 0.3) (layers "F.Cu" "B.Cu") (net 5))
 (segment (start 191.798471 60.96) (end 193.961 58.797471) (width 0.2) (layer "B.Cu") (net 5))
 (segment (start 127 48.26) (end 135.034 48.26) (width 0.2) (layer "B.Cu") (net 5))
 (segment (start 135.034 48.26) (end 147.734 60.96) (width 0.2) (layer "B.Cu") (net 5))
 (segment (start 193.961 58.797471) (end 193.961 41.521) (width 0.2) (layer "B.Cu") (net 5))
 (segment (start 193.961 41.521) (end 193.08 40.64) (width 0.2) (layer "B.Cu") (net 5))
 (segment (start 147.734 60.96) (end 191.798471 60.96) (width 0.2) (layer "B.Cu") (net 5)))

